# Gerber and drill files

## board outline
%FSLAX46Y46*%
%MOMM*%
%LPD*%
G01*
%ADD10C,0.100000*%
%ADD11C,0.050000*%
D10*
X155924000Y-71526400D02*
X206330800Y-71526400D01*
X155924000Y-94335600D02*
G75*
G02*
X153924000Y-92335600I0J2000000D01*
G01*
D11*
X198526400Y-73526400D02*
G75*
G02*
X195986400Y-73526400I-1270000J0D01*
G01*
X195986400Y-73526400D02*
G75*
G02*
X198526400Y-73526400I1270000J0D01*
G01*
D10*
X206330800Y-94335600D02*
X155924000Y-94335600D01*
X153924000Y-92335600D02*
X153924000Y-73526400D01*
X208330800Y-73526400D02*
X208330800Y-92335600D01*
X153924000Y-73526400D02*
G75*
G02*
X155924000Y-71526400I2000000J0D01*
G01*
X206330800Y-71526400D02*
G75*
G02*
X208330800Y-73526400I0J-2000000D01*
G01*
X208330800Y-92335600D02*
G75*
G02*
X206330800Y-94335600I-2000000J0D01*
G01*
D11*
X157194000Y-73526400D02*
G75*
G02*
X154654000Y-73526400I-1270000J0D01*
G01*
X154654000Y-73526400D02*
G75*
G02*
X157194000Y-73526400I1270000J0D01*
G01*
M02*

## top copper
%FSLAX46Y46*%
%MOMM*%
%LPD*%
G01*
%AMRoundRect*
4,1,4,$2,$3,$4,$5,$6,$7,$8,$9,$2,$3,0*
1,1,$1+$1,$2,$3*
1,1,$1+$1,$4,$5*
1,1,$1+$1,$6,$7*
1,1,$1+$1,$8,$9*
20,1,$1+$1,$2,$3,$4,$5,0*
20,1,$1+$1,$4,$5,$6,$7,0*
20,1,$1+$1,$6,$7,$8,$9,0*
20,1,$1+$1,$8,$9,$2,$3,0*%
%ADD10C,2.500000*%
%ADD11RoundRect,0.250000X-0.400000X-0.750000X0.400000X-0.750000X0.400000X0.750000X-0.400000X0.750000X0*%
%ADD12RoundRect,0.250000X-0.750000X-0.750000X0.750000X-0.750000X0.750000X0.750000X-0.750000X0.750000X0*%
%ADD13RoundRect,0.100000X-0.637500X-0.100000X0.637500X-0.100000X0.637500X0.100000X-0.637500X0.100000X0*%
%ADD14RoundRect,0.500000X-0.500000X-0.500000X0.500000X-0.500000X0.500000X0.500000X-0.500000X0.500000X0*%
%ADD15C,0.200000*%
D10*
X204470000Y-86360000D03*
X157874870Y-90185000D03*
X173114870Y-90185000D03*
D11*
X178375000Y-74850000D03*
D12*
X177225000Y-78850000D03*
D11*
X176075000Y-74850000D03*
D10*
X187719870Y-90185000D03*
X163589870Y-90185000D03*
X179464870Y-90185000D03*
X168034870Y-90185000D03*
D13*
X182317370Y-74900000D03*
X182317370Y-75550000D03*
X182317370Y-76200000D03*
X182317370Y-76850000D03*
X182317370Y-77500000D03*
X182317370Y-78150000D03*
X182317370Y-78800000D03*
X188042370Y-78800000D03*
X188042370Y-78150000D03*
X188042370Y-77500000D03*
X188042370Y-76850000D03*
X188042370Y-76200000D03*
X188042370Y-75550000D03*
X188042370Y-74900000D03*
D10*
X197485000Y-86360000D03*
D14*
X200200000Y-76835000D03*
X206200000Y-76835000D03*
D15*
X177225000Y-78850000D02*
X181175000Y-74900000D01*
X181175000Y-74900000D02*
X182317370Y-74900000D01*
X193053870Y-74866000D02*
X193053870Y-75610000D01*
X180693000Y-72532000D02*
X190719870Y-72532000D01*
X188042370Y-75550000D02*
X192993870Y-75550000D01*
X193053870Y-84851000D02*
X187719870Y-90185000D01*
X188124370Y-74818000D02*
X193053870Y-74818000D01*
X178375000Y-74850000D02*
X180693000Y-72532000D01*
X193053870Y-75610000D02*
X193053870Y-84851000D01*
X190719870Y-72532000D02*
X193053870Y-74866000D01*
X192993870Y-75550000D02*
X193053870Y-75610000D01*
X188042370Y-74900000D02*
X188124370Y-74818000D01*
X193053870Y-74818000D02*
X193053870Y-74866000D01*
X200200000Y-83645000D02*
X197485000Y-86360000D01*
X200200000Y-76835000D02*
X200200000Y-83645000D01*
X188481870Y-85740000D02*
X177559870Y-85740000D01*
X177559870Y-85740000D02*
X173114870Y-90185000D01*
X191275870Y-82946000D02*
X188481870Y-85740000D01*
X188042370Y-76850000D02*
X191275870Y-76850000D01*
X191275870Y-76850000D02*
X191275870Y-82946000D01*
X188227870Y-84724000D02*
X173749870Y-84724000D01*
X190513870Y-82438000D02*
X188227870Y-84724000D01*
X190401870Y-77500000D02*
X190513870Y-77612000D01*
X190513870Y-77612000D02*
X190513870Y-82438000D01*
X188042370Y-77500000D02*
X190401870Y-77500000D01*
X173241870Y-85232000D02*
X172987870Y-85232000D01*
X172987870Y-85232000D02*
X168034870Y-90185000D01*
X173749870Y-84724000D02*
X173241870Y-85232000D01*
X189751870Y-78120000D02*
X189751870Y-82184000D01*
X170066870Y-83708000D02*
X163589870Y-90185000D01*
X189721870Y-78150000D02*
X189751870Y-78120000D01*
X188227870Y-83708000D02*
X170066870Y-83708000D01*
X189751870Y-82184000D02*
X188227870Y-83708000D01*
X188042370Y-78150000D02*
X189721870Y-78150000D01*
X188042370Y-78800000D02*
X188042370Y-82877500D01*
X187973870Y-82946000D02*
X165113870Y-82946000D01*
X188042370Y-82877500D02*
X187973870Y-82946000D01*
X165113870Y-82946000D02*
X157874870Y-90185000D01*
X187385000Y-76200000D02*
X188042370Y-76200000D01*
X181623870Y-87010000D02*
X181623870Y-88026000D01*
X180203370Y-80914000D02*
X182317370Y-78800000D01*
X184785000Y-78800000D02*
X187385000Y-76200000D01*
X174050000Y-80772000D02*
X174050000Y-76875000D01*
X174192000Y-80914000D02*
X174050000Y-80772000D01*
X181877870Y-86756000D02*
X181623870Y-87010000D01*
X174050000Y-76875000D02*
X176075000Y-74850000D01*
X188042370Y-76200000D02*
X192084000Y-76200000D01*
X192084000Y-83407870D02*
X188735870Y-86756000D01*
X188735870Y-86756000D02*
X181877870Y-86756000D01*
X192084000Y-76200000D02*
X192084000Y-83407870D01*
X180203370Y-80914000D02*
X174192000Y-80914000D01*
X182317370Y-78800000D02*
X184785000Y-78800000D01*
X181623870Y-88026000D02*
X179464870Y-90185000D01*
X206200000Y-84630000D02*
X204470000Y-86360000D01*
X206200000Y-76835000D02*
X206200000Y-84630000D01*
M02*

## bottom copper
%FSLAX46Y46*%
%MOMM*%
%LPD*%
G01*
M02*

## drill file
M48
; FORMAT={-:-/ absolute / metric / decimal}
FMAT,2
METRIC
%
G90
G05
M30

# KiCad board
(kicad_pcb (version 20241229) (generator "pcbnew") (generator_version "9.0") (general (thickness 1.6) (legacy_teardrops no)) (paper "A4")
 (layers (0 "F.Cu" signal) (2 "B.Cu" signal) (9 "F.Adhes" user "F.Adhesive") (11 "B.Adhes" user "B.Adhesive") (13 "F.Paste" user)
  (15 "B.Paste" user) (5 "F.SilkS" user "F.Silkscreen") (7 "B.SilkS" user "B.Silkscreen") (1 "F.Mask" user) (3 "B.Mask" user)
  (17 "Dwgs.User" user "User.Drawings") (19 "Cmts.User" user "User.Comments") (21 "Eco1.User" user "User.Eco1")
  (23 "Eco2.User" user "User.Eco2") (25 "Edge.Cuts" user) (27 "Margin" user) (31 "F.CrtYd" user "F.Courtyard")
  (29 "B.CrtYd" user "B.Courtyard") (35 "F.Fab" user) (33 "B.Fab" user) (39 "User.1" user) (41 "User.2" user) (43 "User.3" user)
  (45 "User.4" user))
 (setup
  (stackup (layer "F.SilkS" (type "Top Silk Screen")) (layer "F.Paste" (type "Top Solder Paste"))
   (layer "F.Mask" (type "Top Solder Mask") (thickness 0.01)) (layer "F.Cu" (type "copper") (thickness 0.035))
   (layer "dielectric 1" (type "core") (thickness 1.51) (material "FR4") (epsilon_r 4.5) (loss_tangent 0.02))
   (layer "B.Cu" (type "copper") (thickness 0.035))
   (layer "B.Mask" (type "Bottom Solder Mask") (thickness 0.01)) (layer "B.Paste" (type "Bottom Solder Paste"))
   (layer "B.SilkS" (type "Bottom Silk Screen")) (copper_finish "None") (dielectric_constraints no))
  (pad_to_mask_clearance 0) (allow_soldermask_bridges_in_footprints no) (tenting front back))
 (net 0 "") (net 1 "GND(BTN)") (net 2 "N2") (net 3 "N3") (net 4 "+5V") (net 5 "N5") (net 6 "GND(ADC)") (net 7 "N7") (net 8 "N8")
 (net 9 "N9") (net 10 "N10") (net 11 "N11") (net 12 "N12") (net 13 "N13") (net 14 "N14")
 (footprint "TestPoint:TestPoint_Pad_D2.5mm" (layer "F.Cu") (at 204.47 86.36)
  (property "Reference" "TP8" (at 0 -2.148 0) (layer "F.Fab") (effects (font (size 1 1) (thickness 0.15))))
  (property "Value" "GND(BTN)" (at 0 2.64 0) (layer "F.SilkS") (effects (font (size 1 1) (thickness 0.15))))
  (pad "1" smd circle (at 0 0) (size 2.5 2.5) (layers "F.Cu" "F.Mask") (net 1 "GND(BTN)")))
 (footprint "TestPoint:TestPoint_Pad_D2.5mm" (layer "F.Cu") (at 157.87487 90.185)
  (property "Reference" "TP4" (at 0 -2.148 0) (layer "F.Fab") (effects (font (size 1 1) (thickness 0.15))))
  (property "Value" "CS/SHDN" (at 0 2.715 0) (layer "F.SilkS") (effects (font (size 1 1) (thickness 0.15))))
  (pad "1" smd circle (at 0 0) (size 2.5 2.5) (layers "F.Cu" "F.Mask") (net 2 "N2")))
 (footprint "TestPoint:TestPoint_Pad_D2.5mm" (layer "F.Cu") (at 173.11487 90.185)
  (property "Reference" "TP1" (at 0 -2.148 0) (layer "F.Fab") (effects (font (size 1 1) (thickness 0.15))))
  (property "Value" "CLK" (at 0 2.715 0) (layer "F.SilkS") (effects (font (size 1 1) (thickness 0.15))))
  (pad "1" smd circle (at 0 0) (size 2.5 2.5) (layers "F.Cu" "F.Mask") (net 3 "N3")))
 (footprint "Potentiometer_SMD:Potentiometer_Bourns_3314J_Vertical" (layer "F.Cu") (at 177.225 76.85)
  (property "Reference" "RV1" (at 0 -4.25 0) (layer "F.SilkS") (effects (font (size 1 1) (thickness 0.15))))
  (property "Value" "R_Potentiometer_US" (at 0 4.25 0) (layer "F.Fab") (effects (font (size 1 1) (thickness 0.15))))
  (pad "1" smd roundrect (at 1.15 -2) (size 1.3 2) (layers "F.Cu" "F.Mask" "F.Paste") (roundrect_rratio 0.192308) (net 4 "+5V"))
  (pad "2" smd roundrect (at 0 2) (size 2 2) (layers "F.Cu" "F.Mask" "F.Paste") (roundrect_rratio 0.125) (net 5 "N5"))
  (pad "3" smd roundrect (at -1.15 -2) (size 1.3 2) (layers "F.Cu" "F.Mask" "F.Paste") (roundrect_rratio 0.192308) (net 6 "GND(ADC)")))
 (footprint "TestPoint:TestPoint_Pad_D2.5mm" (layer "F.Cu") (at 187.71987 90.185)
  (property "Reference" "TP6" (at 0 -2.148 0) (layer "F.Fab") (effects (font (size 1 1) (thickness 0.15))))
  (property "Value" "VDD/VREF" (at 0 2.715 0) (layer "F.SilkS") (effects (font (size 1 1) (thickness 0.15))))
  (pad "1" smd circle (at 0 0) (size 2.5 2.5) (layers "F.Cu" "F.Mask") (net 4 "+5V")))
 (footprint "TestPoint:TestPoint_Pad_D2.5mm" (layer "F.Cu") (at 163.58987 90.185)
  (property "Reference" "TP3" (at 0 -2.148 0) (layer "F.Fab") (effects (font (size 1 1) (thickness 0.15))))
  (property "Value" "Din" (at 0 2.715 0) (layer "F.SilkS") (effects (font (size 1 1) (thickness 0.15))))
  (pad "1" smd circle (at 0 0) (size 2.5 2.5) (layers "F.Cu" "F.Mask") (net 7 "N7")))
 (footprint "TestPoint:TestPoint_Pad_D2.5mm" (layer "F.Cu") (at 179.46487 90.185)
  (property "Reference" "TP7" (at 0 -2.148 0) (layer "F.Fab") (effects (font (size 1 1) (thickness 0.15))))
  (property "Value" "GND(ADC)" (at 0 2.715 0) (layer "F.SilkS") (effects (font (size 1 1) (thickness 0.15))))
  (pad "1" smd circle (at 0 0) (size 2.5 2.5) (layers "F.Cu" "F.Mask") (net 6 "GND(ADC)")))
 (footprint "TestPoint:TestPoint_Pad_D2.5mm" (layer "F.Cu") (at 168.03487 90.185)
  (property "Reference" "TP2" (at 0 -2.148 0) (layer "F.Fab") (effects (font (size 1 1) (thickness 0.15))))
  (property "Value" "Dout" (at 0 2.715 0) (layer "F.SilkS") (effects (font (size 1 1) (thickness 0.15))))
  (pad "1" smd circle (at 0 0) (size 2.5 2.5) (layers "F.Cu" "F.Mask") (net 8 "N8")))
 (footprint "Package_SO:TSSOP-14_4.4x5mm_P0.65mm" (layer "F.Cu") (at 185.17987 76.85)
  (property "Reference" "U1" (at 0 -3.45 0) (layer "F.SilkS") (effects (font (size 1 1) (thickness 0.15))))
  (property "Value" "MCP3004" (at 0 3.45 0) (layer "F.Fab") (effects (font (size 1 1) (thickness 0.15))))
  (pad "1" smd roundrect (at -2.8625 -1.95) (size 1.475 0.4) (layers "F.Cu" "F.Mask" "F.Paste") (roundrect_rratio 0.25) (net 5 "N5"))
  (pad "2" smd roundrect (at -2.8625 -1.3) (size 1.475 0.4) (layers "F.Cu" "F.Mask" "F.Paste") (roundrect_rratio 0.25) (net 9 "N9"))
  (pad "3" smd roundrect (at -2.8625 -0.65) (size 1.475 0.4) (layers "F.Cu" "F.Mask" "F.Paste") (roundrect_rratio 0.25) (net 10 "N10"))
  (pad "4" smd roundrect (at -2.8625 0) (size 1.475 0.4) (layers "F.Cu" "F.Mask" "F.Paste") (roundrect_rratio 0.25) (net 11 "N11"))
  (pad "5" smd roundrect (at -2.8625 0.65) (size 1.475 0.4) (layers "F.Cu" "F.Mask" "F.Paste") (roundrect_rratio 0.25) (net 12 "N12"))
  (pad "6" smd roundrect (at -2.8625 1.3) (size 1.475 0.4) (layers "F.Cu" "F.Mask" "F.Paste") (roundrect_rratio 0.25) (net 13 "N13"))
  (pad "7" smd roundrect (at -2.8625 1.95) (size 1.475 0.4) (layers "F.Cu" "F.Mask" "F.Paste") (roundrect_rratio 0.25) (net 6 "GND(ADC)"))
  (pad "8" smd roundrect (at 2.8625 1.95) (size 1.475 0.4) (layers "F.Cu" "F.Mask" "F.Paste") (roundrect_rratio 0.25) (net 2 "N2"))
  (pad "9" smd roundrect (at 2.8625 1.3) (size 1.475 0.4) (layers "F.Cu" "F.Mask" "F.Paste") (roundrect_rratio 0.25) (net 7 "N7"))
  (pad "10" smd roundrect (at 2.8625 0.65) (size 1.475 0.4) (layers "F.Cu" "F.Mask" "F.Paste") (roundrect_rratio 0.25) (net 8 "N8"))
  (pad "11" smd roundrect (at 2.8625 0) (size 1.475 0.4) (layers "F.Cu" "F.Mask" "F.Paste") (roundrect_rratio 0.25) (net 3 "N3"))
  (pad "12" smd roundrect (at 2.8625 -0.65) (size 1.475 0.4) (layers "F.Cu" "F.Mask" "F.Paste") (roundrect_rratio 0.25) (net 6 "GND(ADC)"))
  (pad "13" smd roundrect (at 2.8625 -1.3) (size 1.475 0.4) (layers "F.Cu" "F.Mask" "F.Paste") (roundrect_rratio 0.25) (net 4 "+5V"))
  (pad "14" smd roundrect (at 2.8625 -1.95) (size 1.475 0.4) (layers "F.Cu" "F.Mask" "F.Paste") (roundrect_rratio 0.25) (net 4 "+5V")))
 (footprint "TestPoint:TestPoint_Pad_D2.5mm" (layer "F.Cu") (at 197.485 86.36)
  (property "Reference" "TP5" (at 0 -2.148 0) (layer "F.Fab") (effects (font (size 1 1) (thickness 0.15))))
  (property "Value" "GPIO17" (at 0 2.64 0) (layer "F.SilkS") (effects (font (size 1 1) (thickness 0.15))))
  (pad "1" smd circle (at 0 0) (size 2.5 2.5) (layers "F.Cu" "F.Mask") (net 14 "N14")))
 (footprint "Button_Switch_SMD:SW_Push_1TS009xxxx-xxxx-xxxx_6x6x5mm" (layer "F.Cu") (at 203.2 76.835)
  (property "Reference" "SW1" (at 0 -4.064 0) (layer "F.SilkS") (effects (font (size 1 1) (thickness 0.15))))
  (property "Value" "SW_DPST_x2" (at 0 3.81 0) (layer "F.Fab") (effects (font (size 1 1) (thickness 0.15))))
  (pad "1" smd roundrect (at -3 0) (size 2 2) (layers "F.Cu" "F.Mask" "F.Paste") (roundrect_rratio 0.25) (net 14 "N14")
   (thermal_bridge_angle 45))
  (pad "2" smd roundrect (at 3 0) (size 2 2) (layers "F.Cu" "F.Mask" "F.Paste") (roundrect_rratio 0.25) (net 1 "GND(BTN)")
   (thermal_bridge_angle 45)))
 (gr_line (start 155.924 71.5264) (end 206.3308 71.5264) (stroke (width 0.1) (type default)) (layer "Edge.Cuts"))
 (gr_arc (start 155.924 94.3356) (mid 154.509786 93.749814) (end 153.924 92.3356) (stroke (width 0.1) (type default)) (layer "Edge.Cuts"))
 (gr_circle (center 197.2564 73.5264) (end 198.5264 73.5264) (stroke (width 0.05) (type default)) (fill no) (layer "Edge.Cuts"))
 (gr_line (start 206.3308 94.3356) (end 155.924 94.3356) (stroke (width 0.1) (type default)) (layer "Edge.Cuts"))
 (gr_line (start 153.924 92.3356) (end 153.924 73.5264) (stroke (width 0.1) (type default)) (layer "Edge.Cuts"))
 (gr_line (start 208.3308 73.5264) (end 208.3308 92.3356) (stroke (width 0.1) (type default)) (layer "Edge.Cuts"))
 (gr_arc (start 153.924 73.5264) (mid 154.509786 72.112186) (end 155.924 71.5264) (stroke (width 0.1) (type default)) (layer "Edge.Cuts"))
 (gr_arc (start 206.3308 71.5264) (mid 207.745014 72.112186) (end 208.3308 73.5264) (stroke (width 0.1) (type default)) (layer "Edge.Cuts"))
 (gr_arc (start 208.3308 92.3356) (mid 207.745014 93.749814) (end 206.3308 94.3356) (stroke (width 0.1) (type default)) (layer "Edge.Cuts"))
 (gr_circle (center 155.924 73.5264) (end 157.194 73.5264) (stroke (width 0.05) (type default)) (fill no) (layer "Edge.Cuts"))
 (segment (start 177.225 78.85) (end 181.175 74.9) (width 0.2) (layer "F.Cu") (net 5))
 (segment (start 181.175 74.9) (end 182.31737 74.9) (width 0.2) (layer "F.Cu") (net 5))
 (segment (start 193.05387 74.866) (end 193.05387 75.61) (width 0.2) (layer "F.Cu") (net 4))
 (segment (start 180.693 72.532) (end 190.71987 72.532) (width 0.2) (layer "F.Cu") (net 4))
 (segment (start 188.04237 75.55) (end 192.99387 75.55) (width 0.2) (layer "F.Cu") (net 4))
 (segment (start 193.05387 84.851) (end 187.71987 90.185) (width 0.2) (layer "F.Cu") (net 4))
 (segment (start 188.12437 74.818) (end 193.05387 74.818) (width 0.2) (layer "F.Cu") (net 4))
 (segment (start 178.375 74.85) (end 180.693 72.532) (width 0.2) (layer "F.Cu") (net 4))
 (segment (start 193.05387 75.61) (end 193.05387 84.851) (width 0.2) (layer "F.Cu") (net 4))
 (segment (start 190.71987 72.532) (end 193.05387 74.866) (width 0.2) (layer "F.Cu") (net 4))
 (segment (start 192.99387 75.55) (end 193.05387 75.61) (width 0.2) (layer "F.Cu") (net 4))
 (segment (start 188.04237 74.9) (end 188.12437 74.818) (width 0.2) (layer "F.Cu") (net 4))
 (segment (start 193.05387 74.818) (end 193.05387 74.866) (width 0.2) (layer "F.Cu") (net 4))
 (segment (start 200.2 83.645) (end 197.485 86.36) (width 0.2) (layer "F.Cu") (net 14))
 (segment (start 200.2 76.835) (end 200.2 83.645) (width 0.2) (layer "F.Cu") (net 14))
 (segment (start 188.48187 85.74) (end 177.55987 85.74) (width 0.2) (layer "F.Cu") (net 3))
 (segment (start 177.55987 85.74) (end 173.11487 90.185) (width 0.2) (layer "F.Cu") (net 3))
 (segment (start 191.27587 82.946) (end 188.48187 85.74) (width 0.2) (layer "F.Cu") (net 3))
 (segment (start 188.04237 76.85) (end 191.27587 76.85) (width 0.2) (layer "F.Cu") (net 3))
 (segment (start 191.27587 76.85) (end 191.27587 82.946) (width 0.2) (layer "F.Cu") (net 3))
 (segment (start 188.22787 84.724) (end 173.74987 84.724) (width 0.2) (layer "F.Cu") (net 8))
 (segment (start 190.51387 82.438) (end 188.22787 84.724) (width 0.2) (layer "F.Cu") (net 8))
 (segment (start 190.40187 77.5) (end 190.51387 77.612) (width 0.2) (layer "F.Cu") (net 8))
 (segment (start 190.51387 77.612) (end 190.51387 82.438) (width 0.2) (layer "F.Cu") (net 8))
 (segment (start 188.04237 77.5) (end 190.40187 77.5) (width 0.2) (layer "F.Cu") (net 8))
 (segment (start 173.24187 85.232) (end 172.98787 85.232) (width 0.2) (layer "F.Cu") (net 8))
 (segment (start 172.98787 85.232) (end 168.03487 90.185) (width 0.2) (layer "F.Cu") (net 8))
 (segment (start 173.74987 84.724) (end 173.24187 85.232) (width 0.2) (layer "F.Cu") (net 8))
 (segment (start 189.75187 78.12) (end 189.75187 82.184) (width 0.2) (layer "F.Cu") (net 7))
 (segment (start 170.06687 83.708) (end 163.58987 90.185) (width 0.2) (layer "F.Cu") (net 7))
 (segment (start 189.72187 78.15) (end 189.75187 78.12) (width 0.2) (layer "F.Cu") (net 7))
 (segment (start 188.22787 83.708) (end 170.06687 83.708) (width 0.2) (layer "F.Cu") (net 7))
 (segment (start 189.75187 82.184) (end 188.22787 83.708) (width 0.2) (layer "F.Cu") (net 7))
 (segment (start 188.04237 78.15) (end 189.72187 78.15) (width 0.2) (layer "F.Cu") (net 7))
 (segment (start 188.04237 78.8) (end 188.04237 82.8775) (width 0.2) (layer "F.Cu") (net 2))
 (segment (start 187.97387 82.946) (end 165.11387 82.946) (width 0.2) (layer "F.Cu") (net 2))
 (segment (start 188.04237 82.8775) (end 187.97387 82.946) (width 0.2) (layer "F.Cu") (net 2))
 (segment (start 165.11387 82.946) (end 157.87487 90.185) (width 0.2) (layer "F.Cu") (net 2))
 (segment (start 187.385 76.2) (end 188.04237 76.2) (width 0.2) (layer "F.Cu") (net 6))
 (segment (start 181.62387 87.01) (end 181.62387 88.026) (width 0.2) (layer "F.Cu") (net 6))
 (segment (start 180.20337 80.914) (end 182.31737 78.8) (width 0.2) (layer "F.Cu") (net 6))
 (segment (start 184.785 78.8) (end 187.385 76.2) (width 0.2) (layer "F.Cu") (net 6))
 (segment (start 174.05 80.772) (end 174.05 76.875) (width 0.2) (layer "F.Cu") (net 6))
 (segment (start 174.192 80.914) (end 174.05 80.772) (width 0.2) (layer "F.Cu") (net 6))
 (segment (start 181.87787 86.756) (end 181.62387 87.01) (width 0.2) (layer "F.Cu") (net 6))
 (segment (start 174.05 76.875) (end 176.075 74.85) (width 0.2) (layer "F.Cu") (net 6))
 (segment (start 188.04237 76.2) (end 192.084 76.2) (width 0.2) (layer "F.Cu") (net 6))
 (segment (start 192.084 83.40787) (end 188.73587 86.756) (width 0.2) (layer "F.Cu") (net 6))
 (segment (start 188.73587 86.756) (end 181.87787 86.756) (width 0.2) (layer "F.Cu") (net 6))
 (segment (start 192.084 76.2) (end 192.084 83.40787) (width 0.2) (layer "F.Cu") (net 6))
 (segment (start 180.20337 80.914) (end 174.192 80.914) (width 0.2) (layer "F.Cu") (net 6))
 (segment (start 182.31737 78.8) (end 184.785 78.8) (width 0.2) (layer "F.Cu") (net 6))
 (segment (start 181.62387 88.026) (end 179.46487 90.185) (width 0.2) (layer "F.Cu") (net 6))
 (segment (start 206.2 84.63) (end 204.47 86.36) (width 0.2) (layer "F.Cu") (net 1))
 (segment (start 206.2 76.835) (end 206.2 84.63) (width 0.2) (layer "F.Cu") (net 1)))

